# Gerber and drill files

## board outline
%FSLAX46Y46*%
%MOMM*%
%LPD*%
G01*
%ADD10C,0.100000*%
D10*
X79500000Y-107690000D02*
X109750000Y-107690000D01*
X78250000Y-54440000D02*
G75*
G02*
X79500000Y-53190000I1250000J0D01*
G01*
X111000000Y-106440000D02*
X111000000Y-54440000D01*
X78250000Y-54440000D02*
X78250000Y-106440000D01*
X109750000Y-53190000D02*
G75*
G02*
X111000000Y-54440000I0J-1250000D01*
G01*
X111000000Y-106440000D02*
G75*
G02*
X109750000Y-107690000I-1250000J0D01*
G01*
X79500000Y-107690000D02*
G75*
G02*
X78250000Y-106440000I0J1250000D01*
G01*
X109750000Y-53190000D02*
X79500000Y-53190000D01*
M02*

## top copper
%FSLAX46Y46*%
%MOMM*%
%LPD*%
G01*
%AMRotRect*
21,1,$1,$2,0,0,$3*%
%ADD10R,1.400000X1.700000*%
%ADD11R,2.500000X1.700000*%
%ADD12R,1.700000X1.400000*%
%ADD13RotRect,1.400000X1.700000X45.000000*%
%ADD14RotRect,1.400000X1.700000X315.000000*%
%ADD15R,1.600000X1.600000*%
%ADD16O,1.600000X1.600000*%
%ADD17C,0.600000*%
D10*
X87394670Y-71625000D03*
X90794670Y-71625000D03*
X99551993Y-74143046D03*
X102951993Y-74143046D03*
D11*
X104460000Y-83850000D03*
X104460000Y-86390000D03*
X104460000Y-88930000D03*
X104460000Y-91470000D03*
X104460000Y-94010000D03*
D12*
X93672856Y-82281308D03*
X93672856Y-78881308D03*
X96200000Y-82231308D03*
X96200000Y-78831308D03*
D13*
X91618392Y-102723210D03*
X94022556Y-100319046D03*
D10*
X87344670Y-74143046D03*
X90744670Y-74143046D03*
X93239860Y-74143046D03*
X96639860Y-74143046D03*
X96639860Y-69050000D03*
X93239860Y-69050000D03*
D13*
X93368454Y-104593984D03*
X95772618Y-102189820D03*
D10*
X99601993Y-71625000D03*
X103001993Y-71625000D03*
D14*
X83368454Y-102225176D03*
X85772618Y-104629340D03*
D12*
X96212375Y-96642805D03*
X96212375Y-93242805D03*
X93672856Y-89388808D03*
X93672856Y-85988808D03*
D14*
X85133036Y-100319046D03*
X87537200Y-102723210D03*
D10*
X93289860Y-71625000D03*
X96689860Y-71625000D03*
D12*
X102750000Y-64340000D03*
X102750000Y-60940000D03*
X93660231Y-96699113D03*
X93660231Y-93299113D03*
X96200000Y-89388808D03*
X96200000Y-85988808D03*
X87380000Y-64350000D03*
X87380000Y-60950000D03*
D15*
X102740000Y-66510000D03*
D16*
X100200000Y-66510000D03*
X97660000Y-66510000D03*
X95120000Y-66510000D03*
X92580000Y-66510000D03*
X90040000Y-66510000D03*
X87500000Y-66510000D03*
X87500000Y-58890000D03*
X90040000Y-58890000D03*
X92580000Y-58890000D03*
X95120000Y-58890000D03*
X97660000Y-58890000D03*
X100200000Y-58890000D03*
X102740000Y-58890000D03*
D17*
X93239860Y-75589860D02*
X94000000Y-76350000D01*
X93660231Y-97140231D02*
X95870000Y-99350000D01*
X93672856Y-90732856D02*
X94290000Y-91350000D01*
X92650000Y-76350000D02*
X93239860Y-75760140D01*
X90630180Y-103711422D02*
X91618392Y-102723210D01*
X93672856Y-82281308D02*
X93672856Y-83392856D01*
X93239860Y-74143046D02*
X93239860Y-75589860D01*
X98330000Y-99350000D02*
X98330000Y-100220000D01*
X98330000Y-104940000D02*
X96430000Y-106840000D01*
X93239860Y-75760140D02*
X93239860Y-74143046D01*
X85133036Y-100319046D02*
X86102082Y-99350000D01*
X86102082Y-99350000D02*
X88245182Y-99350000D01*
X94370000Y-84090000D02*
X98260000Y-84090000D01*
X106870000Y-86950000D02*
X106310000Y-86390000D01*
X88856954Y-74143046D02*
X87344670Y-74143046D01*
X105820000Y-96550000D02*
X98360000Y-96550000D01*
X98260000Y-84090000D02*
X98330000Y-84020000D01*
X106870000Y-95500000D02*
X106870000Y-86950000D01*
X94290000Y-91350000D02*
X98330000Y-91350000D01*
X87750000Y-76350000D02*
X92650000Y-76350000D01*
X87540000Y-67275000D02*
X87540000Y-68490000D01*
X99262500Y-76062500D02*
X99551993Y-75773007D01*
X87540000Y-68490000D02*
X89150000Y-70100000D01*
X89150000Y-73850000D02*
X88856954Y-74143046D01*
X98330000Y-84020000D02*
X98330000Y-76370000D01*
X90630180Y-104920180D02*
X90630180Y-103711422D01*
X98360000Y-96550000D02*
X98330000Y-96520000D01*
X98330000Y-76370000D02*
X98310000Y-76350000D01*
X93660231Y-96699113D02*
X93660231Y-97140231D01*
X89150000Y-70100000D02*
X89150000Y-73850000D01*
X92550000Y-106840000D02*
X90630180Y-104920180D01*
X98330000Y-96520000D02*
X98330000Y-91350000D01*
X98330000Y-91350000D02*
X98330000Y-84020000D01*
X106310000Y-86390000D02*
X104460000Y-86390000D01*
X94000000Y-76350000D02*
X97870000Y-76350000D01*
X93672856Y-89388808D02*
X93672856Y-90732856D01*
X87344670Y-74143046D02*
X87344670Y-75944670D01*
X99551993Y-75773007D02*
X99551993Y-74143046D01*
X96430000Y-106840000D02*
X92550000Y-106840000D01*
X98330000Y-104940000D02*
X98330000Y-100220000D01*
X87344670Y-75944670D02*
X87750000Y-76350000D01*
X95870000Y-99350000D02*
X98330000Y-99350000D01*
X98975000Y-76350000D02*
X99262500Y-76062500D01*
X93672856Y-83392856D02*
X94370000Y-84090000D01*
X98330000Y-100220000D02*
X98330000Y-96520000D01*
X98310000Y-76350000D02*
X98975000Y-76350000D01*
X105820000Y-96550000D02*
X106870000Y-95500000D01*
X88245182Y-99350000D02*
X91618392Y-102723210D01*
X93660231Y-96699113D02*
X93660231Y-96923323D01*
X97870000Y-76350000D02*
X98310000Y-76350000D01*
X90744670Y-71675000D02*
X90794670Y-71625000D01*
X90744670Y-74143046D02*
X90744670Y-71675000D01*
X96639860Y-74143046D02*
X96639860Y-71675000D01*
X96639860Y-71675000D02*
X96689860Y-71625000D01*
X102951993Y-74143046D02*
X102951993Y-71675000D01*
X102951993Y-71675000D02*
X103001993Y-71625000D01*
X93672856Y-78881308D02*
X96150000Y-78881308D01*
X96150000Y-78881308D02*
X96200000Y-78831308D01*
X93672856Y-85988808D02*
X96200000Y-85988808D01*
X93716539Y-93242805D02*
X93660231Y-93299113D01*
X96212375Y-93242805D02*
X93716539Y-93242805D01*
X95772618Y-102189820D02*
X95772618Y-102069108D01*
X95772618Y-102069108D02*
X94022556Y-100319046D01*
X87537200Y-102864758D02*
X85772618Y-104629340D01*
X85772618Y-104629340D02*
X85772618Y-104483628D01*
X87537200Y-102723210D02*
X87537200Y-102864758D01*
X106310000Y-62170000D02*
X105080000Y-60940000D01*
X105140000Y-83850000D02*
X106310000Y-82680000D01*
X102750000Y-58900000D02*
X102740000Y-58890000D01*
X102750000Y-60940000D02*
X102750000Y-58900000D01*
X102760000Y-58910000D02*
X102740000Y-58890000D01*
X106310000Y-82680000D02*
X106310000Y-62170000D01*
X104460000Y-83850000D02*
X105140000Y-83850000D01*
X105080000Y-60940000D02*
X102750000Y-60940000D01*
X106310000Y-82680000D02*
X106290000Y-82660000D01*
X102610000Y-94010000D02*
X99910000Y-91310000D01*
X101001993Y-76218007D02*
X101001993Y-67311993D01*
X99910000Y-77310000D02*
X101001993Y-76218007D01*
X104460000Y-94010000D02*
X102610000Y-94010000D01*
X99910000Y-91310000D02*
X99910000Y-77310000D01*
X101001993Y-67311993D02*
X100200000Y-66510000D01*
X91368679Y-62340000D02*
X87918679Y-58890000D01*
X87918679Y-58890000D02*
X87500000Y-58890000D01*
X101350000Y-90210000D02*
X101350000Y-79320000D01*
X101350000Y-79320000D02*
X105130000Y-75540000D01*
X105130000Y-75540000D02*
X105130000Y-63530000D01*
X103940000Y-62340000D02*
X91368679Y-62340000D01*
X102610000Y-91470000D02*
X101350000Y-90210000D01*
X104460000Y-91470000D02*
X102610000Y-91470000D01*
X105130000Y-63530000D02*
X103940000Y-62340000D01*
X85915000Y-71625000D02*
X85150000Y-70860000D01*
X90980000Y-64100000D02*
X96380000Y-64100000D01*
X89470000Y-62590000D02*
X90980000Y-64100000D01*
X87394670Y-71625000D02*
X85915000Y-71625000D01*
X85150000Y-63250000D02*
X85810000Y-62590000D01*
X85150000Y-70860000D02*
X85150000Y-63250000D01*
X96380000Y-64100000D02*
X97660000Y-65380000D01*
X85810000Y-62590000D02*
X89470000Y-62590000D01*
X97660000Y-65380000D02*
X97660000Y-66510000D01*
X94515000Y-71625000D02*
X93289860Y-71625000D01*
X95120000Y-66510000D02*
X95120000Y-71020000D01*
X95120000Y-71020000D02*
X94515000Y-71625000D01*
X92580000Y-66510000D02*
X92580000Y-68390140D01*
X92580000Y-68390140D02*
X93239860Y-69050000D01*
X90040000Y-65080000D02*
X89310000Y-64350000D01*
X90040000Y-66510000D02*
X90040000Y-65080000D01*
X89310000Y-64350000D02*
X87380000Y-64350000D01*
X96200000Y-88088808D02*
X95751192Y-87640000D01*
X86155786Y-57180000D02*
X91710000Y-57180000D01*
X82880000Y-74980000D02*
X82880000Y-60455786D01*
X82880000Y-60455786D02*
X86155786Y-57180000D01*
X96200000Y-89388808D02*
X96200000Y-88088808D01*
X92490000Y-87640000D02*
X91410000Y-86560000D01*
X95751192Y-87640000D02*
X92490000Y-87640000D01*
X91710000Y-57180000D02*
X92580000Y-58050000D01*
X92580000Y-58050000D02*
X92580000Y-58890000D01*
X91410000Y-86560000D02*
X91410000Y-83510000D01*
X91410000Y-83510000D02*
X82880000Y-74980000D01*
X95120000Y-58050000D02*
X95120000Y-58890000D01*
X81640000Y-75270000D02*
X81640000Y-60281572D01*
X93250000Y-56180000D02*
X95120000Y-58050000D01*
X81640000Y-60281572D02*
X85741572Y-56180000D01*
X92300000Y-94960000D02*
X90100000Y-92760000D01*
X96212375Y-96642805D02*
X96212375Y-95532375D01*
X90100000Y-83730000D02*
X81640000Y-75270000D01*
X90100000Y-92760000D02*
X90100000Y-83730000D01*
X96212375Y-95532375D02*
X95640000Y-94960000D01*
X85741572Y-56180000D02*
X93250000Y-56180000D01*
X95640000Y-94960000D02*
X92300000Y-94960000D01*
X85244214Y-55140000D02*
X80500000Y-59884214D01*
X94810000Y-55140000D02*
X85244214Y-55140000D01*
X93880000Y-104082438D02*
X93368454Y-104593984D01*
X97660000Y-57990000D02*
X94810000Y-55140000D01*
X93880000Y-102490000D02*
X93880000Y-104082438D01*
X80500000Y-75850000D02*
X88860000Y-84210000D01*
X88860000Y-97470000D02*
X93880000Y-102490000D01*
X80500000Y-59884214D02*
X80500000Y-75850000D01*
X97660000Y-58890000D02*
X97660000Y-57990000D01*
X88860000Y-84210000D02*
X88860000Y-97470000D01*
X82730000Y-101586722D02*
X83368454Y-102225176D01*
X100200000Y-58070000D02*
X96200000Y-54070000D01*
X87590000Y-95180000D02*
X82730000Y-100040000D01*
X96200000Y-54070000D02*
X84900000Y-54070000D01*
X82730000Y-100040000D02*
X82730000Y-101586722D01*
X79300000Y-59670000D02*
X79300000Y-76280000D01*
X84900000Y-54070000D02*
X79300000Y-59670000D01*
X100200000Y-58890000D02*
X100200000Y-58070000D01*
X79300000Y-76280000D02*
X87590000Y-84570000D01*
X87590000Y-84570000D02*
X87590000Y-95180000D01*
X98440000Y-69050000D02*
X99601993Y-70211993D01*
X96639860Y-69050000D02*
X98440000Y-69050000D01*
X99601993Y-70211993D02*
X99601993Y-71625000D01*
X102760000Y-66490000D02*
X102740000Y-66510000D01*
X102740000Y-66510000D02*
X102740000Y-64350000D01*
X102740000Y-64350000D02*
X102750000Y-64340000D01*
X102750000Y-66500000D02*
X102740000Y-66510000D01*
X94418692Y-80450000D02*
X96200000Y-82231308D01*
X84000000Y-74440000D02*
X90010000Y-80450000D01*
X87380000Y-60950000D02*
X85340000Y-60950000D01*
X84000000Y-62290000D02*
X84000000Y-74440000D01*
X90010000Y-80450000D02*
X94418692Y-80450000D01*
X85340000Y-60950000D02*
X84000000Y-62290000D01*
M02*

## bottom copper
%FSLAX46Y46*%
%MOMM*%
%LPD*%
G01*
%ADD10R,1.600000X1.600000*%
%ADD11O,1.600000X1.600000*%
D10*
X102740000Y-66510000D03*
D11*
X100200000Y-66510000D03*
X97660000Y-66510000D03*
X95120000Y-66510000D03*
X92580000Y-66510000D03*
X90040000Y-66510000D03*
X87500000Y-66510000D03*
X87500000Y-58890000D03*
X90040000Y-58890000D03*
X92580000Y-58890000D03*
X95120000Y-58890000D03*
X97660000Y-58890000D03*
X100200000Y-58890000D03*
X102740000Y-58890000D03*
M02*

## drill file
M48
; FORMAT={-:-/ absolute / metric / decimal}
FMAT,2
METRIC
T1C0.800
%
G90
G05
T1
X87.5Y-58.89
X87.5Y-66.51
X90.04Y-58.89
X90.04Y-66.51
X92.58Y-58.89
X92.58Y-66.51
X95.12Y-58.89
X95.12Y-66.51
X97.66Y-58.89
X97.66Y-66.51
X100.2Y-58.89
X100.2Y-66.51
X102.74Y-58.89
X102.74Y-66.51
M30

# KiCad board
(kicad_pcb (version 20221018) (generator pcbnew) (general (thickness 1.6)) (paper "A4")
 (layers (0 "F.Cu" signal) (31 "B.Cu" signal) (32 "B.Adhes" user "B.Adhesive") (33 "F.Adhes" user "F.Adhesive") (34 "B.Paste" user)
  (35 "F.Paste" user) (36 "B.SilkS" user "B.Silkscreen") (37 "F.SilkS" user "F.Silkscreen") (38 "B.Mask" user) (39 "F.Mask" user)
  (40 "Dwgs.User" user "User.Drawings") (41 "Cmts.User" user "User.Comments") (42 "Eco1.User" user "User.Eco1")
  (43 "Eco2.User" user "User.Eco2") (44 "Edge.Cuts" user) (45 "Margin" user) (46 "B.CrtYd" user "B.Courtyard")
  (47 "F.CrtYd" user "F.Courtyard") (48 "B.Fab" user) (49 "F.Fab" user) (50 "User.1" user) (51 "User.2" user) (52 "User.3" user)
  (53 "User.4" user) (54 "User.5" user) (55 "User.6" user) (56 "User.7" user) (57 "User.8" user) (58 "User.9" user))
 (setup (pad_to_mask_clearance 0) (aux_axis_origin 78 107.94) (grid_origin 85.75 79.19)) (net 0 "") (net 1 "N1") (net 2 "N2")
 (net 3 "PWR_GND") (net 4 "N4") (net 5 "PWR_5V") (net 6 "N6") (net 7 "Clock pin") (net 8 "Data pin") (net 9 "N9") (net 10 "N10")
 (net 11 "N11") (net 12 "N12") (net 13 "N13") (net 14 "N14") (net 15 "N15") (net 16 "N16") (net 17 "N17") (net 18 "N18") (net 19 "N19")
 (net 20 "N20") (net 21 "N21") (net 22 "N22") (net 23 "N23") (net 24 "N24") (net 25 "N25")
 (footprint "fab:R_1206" (layer "F.Cu") (at 89.09467 71.625)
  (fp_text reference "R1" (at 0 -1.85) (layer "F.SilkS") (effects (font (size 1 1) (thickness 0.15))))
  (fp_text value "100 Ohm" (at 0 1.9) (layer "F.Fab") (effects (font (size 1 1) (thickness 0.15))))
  (pad "1" smd rect (at -1.7 0) (size 1.4 1.7) (layers "F.Cu" "F.Paste" "F.Mask") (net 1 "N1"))
  (pad "2" smd rect (at 1.7 0) (size 1.4 1.7) (layers "F.Cu" "F.Paste" "F.Mask") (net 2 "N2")))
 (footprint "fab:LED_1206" (layer "F.Cu") (at 101.251993 74.143046)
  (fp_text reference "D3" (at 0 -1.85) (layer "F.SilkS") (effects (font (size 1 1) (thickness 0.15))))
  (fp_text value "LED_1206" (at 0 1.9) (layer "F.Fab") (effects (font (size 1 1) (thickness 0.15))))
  (pad "1" smd rect (at -1.7 0) (size 1.4 1.7) (layers "F.Cu" "F.Paste" "F.Mask") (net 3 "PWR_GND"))
  (pad "2" smd rect (at 1.7 0) (size 1.4 1.7) (layers "F.Cu" "F.Paste" "F.Mask") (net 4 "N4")))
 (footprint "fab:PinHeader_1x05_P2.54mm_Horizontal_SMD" (layer "F.Cu") (at 104.46 83.85)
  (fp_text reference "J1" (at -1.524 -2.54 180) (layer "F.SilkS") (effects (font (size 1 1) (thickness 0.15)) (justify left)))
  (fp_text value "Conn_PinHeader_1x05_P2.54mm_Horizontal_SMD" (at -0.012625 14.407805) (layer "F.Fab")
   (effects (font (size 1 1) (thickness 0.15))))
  (pad "1" smd rect (at 0 0) (size 2.5 1.7) (layers "F.Cu" "F.Paste" "F.Mask") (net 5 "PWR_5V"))
  (pad "2" smd rect (at 0 2.54) (size 2.5 1.7) (layers "F.Cu" "F.Paste" "F.Mask") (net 3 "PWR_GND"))
  (pad "3" smd rect (at 0 5.08) (size 2.5 1.7) (layers "F.Cu" "F.Paste" "F.Mask") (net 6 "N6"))
  (pad "4" smd rect (at 0 7.62) (size 2.5 1.7) (layers "F.Cu" "F.Paste" "F.Mask") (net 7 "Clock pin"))
  (pad "5" smd rect (at 0 10.16) (size 2.5 1.7) (layers "F.Cu" "F.Paste" "F.Mask") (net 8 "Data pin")))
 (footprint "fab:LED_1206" (layer "F.Cu") (at 93.672856 80.581308 90)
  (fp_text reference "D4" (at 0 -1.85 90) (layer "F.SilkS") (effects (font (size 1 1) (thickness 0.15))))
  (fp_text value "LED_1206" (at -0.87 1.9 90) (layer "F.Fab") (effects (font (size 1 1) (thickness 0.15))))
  (pad "1" smd rect (at -1.7 0 90) (size 1.4 1.7) (layers "F.Cu" "F.Paste" "F.Mask") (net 3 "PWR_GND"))
  (pad "2" smd rect (at 1.7 0 90) (size 1.4 1.7) (layers "F.Cu" "F.Paste" "F.Mask") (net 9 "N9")))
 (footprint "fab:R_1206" (layer "F.Cu") (at 96.2 80.531308 90)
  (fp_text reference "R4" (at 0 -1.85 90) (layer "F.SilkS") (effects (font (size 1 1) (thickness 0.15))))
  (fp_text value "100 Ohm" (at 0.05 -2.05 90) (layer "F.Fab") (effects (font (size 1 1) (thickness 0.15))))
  (pad "1" smd rect (at -1.7 0 90) (size 1.4 1.7) (layers "F.Cu" "F.Paste" "F.Mask") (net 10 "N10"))
  (pad "2" smd rect (at 1.7 0 90) (size 1.4 1.7) (layers "F.Cu" "F.Paste" "F.Mask") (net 9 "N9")))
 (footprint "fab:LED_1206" (layer "F.Cu") (at 92.820474 101.521128 45)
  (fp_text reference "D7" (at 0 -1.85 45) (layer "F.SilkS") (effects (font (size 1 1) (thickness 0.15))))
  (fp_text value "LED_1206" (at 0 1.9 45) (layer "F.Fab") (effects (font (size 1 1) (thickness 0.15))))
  (pad "1" smd rect (at -1.7 0 45) (size 1.4 1.7) (layers "F.Cu" "F.Paste" "F.Mask") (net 3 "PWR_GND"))
  (pad "2" smd rect (at 1.7 0 45) (size 1.4 1.7) (layers "F.Cu" "F.Paste" "F.Mask") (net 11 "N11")))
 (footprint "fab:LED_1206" (layer "F.Cu") (at 89.04467 74.143046)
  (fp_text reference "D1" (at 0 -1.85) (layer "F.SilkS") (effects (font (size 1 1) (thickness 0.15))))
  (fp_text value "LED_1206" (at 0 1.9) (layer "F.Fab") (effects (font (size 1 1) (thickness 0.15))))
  (pad "1" smd rect (at -1.7 0) (size 1.4 1.7) (layers "F.Cu" "F.Paste" "F.Mask") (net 3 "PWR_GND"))
  (pad "2" smd rect (at 1.7 0) (size 1.4 1.7) (layers "F.Cu" "F.Paste" "F.Mask") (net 2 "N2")))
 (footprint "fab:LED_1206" (layer "F.Cu") (at 94.93986 74.143046)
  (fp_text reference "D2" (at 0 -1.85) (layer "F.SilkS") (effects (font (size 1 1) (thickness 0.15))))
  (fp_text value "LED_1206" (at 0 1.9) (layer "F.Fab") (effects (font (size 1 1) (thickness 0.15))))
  (pad "1" smd rect (at -1.7 0) (size 1.4 1.7) (layers "F.Cu" "F.Paste" "F.Mask") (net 3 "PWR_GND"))
  (pad "2" smd rect (at 1.7 0) (size 1.4 1.7) (layers "F.Cu" "F.Paste" "F.Mask") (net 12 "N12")))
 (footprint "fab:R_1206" (layer "F.Cu") (at 94.93986 69.05 180)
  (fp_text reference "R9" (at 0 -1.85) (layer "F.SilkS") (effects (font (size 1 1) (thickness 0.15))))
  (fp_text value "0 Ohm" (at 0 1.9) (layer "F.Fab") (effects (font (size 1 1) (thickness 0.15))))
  (pad "1" smd rect (at -1.7 0 180) (size 1.4 1.7) (layers "F.Cu" "F.Paste" "F.Mask") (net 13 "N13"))
  (pad "2" smd rect (at 1.7 0 180) (size 1.4 1.7) (layers "F.Cu" "F.Paste" "F.Mask") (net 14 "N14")))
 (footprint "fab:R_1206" (layer "F.Cu") (at 94.570536 103.391902 45)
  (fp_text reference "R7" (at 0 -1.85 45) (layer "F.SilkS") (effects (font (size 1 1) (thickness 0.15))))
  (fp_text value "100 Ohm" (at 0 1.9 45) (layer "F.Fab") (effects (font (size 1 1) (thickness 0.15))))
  (pad "1" smd rect (at -1.7 0 45) (size 1.4 1.7) (layers "F.Cu" "F.Paste" "F.Mask") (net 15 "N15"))
  (pad "2" smd rect (at 1.7 0 45) (size 1.4 1.7) (layers "F.Cu" "F.Paste" "F.Mask") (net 11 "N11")))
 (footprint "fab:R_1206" (layer "F.Cu") (at 101.301993 71.625)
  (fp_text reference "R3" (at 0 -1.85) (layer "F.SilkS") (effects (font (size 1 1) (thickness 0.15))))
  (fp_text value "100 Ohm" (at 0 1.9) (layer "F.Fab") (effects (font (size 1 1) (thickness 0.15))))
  (pad "1" smd rect (at -1.7 0) (size 1.4 1.7) (layers "F.Cu" "F.Paste" "F.Mask") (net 14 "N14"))
  (pad "2" smd rect (at 1.7 0) (size 1.4 1.7) (layers "F.Cu" "F.Paste" "F.Mask") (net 4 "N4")))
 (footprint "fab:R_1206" (layer "F.Cu") (at 84.570536 103.427258 -45)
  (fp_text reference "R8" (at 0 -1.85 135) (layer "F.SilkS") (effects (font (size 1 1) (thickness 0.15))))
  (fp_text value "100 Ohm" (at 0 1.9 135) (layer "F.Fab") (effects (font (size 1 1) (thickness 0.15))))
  (pad "1" smd rect (at -1.7 0 315) (size 1.4 1.7) (layers "F.Cu" "F.Paste" "F.Mask") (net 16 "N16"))
  (pad "2" smd rect (at 1.7 0 315) (size 1.4 1.7) (layers "F.Cu" "F.Paste" "F.Mask") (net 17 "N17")))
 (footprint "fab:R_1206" (layer "F.Cu") (at 96.212375 94.942805 90)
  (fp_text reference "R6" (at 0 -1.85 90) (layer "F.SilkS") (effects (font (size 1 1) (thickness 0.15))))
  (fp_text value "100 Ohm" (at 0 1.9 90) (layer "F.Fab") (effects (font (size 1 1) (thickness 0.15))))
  (pad "1" smd rect (at -1.7 0 90) (size 1.4 1.7) (layers "F.Cu" "F.Paste" "F.Mask") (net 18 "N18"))
  (pad "2" smd rect (at 1.7 0 90) (size 1.4 1.7) (layers "F.Cu" "F.Paste" "F.Mask") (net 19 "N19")))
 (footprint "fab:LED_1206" (layer "F.Cu") (at 93.672856 87.688808 90)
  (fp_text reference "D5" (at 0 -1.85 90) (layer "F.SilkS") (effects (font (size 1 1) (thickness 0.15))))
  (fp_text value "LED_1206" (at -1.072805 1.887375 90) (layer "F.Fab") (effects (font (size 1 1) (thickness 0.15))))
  (pad "1" smd rect (at -1.7 0 90) (size 1.4 1.7) (layers "F.Cu" "F.Paste" "F.Mask") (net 3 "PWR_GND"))
  (pad "2" smd rect (at 1.7 0 90) (size 1.4 1.7) (layers "F.Cu" "F.Paste" "F.Mask") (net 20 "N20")))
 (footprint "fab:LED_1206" (layer "F.Cu") (at 86.335118 101.521128 -45)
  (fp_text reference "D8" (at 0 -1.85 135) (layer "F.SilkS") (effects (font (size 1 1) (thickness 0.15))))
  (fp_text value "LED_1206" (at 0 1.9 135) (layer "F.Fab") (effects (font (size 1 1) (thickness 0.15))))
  (pad "1" smd rect (at -1.7 0 315) (size 1.4 1.7) (layers "F.Cu" "F.Paste" "F.Mask") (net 3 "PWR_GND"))
  (pad "2" smd rect (at 1.7 0 315) (size 1.4 1.7) (layers "F.Cu" "F.Paste" "F.Mask") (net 17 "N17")))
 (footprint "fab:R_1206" (layer "F.Cu") (at 94.98986 71.625)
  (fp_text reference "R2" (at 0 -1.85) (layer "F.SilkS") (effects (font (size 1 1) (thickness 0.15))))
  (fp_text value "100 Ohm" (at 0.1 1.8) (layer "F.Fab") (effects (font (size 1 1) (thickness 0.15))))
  (pad "1" smd rect (at -1.7 0) (size 1.4 1.7) (layers "F.Cu" "F.Paste" "F.Mask") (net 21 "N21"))
  (pad "2" smd rect (at 1.7 0) (size 1.4 1.7) (layers "F.Cu" "F.Paste" "F.Mask") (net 12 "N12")))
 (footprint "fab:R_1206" (layer "F.Cu") (at 102.75 62.64 90)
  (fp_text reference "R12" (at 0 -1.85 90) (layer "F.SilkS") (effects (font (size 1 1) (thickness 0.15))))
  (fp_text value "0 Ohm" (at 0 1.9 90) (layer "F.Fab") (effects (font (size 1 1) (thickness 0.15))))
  (pad "1" smd rect (at -1.7 0 90) (size 1.4 1.7) (layers "F.Cu" "F.Paste" "F.Mask") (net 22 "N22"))
  (pad "2" smd rect (at 1.7 0 90) (size 1.4 1.7) (layers "F.Cu" "F.Paste" "F.Mask") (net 5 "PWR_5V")))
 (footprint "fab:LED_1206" (layer "F.Cu") (at 93.660231 94.999113 90)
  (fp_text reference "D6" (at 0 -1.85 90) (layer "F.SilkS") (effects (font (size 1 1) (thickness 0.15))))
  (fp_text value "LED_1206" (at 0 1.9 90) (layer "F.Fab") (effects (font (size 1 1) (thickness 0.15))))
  (pad "1" smd rect (at -1.7 0 90) (size 1.4 1.7) (layers "F.Cu" "F.Paste" "F.Mask") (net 3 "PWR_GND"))
  (pad "2" smd rect (at 1.7 0 90) (size 1.4 1.7) (layers "F.Cu" "F.Paste" "F.Mask") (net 19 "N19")))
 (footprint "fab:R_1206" (layer "F.Cu") (at 96.2 87.688808 90)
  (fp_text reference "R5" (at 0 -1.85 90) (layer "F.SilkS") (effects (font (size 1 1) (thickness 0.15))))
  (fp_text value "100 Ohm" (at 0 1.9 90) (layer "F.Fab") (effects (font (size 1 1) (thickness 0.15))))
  (pad "1" smd rect (at -1.7 0 90) (size 1.4 1.7) (layers "F.Cu" "F.Paste" "F.Mask") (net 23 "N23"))
  (pad "2" smd rect (at 1.7 0 90) (size 1.4 1.7) (layers "F.Cu" "F.Paste" "F.Mask") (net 20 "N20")))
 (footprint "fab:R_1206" (layer "F.Cu") (at 87.38 62.65 90)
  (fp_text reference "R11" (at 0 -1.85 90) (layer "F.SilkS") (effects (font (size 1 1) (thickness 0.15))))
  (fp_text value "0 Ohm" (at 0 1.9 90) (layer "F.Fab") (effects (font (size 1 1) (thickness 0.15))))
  (pad "1" smd rect (at -1.7 0 90) (size 1.4 1.7) (layers "F.Cu" "F.Paste" "F.Mask") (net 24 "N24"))
  (pad "2" smd rect (at 1.7 0 90) (size 1.4 1.7) (layers "F.Cu" "F.Paste" "F.Mask") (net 10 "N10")))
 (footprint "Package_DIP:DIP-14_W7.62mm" (layer "B.Cu") (at 102.74 66.51 90)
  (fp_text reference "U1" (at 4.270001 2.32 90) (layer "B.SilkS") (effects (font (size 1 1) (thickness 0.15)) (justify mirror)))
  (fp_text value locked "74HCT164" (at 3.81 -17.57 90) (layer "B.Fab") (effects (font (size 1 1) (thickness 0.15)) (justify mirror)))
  (pad "1" thru_hole rect (at 0 0 90) (size 1.6 1.6) (drill 0.8) (layers "*.Cu" "*.Mask") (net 22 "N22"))
  (pad "2" thru_hole oval (at 0 -2.54 90) (size 1.6 1.6) (drill 0.8) (layers "*.Cu" "*.Mask") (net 8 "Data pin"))
  (pad "3" thru_hole oval (at 0 -5.08 90) (size 1.6 1.6) (drill 0.8) (layers "*.Cu" "*.Mask") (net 1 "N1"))
  (pad "4" thru_hole oval (at 0 -7.62 90) (size 1.6 1.6) (drill 0.8) (layers "*.Cu" "*.Mask") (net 21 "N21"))
  (pad "5" thru_hole oval (at 0 -10.16 90) (size 1.6 1.6) (drill 0.8) (layers "*.Cu" "*.Mask") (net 13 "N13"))
  (pad "6" thru_hole oval (at 0 -12.7 90) (size 1.6 1.6) (drill 0.8) (layers "*.Cu" "*.Mask") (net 24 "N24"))
  (pad "7" thru_hole oval (at 0 -15.24 90) (size 1.6 1.6) (drill 0.8) (layers "*.Cu" "*.Mask") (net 3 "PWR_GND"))
  (pad "8" thru_hole oval (at 7.62 -15.24 90) (size 1.6 1.6) (drill 0.8) (layers "*.Cu" "*.Mask") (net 7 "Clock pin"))
  (pad "9" thru_hole oval (at 7.62 -12.7 90) (size 1.6 1.6) (drill 0.8) (layers "*.Cu" "*.Mask") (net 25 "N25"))
  (pad "10" thru_hole oval (at 7.62 -10.16 90) (size 1.6 1.6) (drill 0.8) (layers "*.Cu" "*.Mask") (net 23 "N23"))
  (pad "11" thru_hole oval (at 7.62 -7.62 90) (size 1.6 1.6) (drill 0.8) (layers "*.Cu" "*.Mask") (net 18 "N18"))
  (pad "12" thru_hole oval (at 7.62 -5.08 90) (size 1.6 1.6) (drill 0.8) (layers "*.Cu" "*.Mask") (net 15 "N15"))
  (pad "13" thru_hole oval (at 7.62 -2.54 90) (size 1.6 1.6) (drill 0.8) (layers "*.Cu" "*.Mask") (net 16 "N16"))
  (pad "14" thru_hole oval (at 7.62 0 90) (size 1.6 1.6) (drill 0.8) (layers "*.Cu" "*.Mask") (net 5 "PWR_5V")))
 (gr_line (start 79.5 107.69) (end 109.75 107.69) (stroke (width 0.1) (type default)) (layer "Edge.Cuts"))
 (gr_arc (start 78.25 54.44) (mid 78.616117 53.556117) (end 79.5 53.19) (stroke (width 0.1) (type default)) (layer "Edge.Cuts"))
 (gr_line (start 111 106.44) (end 111 54.44) (stroke (width 0.1) (type default)) (layer "Edge.Cuts"))
 (gr_line (start 78.25 54.44) (end 78.25 106.44) (stroke (width 0.1) (type default)) (layer "Edge.Cuts"))
 (gr_arc (start 109.75 53.19) (mid 110.633883 53.556117) (end 111 54.44) (stroke (width 0.1) (type default)) (layer "Edge.Cuts"))
 (gr_arc (start 111 106.44) (mid 110.633883 107.323883) (end 109.75 107.69) (stroke (width 0.1) (type default)) (layer "Edge.Cuts"))
 (gr_arc (start 79.5 107.69) (mid 78.616117 107.323883) (end 78.25 106.44) (stroke (width 0.1) (type default)) (layer "Edge.Cuts"))
 (gr_line (start 109.75 53.19) (end 79.5 53.19) (stroke (width 0.1) (type default)) (layer "Edge.Cuts"))
 (segment (start 93.23986 75.58986) (end 94 76.35) (width 0.6) (layer "F.Cu") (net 3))
 (segment (start 93.660231 97.140231) (end 95.87 99.35) (width 0.6) (layer "F.Cu") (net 3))
 (segment (start 93.672856 90.732856) (end 94.29 91.35) (width 0.6) (layer "F.Cu") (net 3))
 (segment (start 92.65 76.35) (end 93.23986 75.76014) (width 0.6) (layer "F.Cu") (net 3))
 (segment (start 90.63018 103.711422) (end 91.618392 102.72321) (width 0.6) (layer "F.Cu") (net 3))
 (segment (start 93.672856 82.281308) (end 93.672856 83.392856) (width 0.6) (layer "F.Cu") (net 3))
 (segment (start 93.23986 74.143046) (end 93.23986 75.58986) (width 0.6) (layer "F.Cu") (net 3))
 (segment (start 98.33 99.35) (end 98.33 100.22) (width 0.6) (layer "F.Cu") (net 3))
 (segment (start 98.33 104.94) (end 96.43 106.84) (width 0.6) (layer "F.Cu") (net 3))
 (segment (start 93.23986 75.76014) (end 93.23986 74.143046) (width 0.6) (layer "F.Cu") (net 3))
 (segment (start 85.133036 100.319046) (end 86.102082 99.35) (width 0.6) (layer "F.Cu") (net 3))
 (segment (start 86.102082 99.35) (end 88.245182 99.35) (width 0.6) (layer "F.Cu") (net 3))
 (segment (start 94.37 84.09) (end 98.26 84.09) (width 0.6) (layer "F.Cu") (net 3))
 (segment (start 106.87 86.95) (end 106.31 86.39) (width 0.6) (layer "F.Cu") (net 3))
 (segment (start 88.856954 74.143046) (end 87.34467 74.143046) (width 0.6) (layer "F.Cu") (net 3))
 (segment (start 105.82 96.55) (end 98.36 96.55) (width 0.6) (layer "F.Cu") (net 3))
 (segment (start 98.26 84.09) (end 98.33 84.02) (width 0.6) (layer "F.Cu") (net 3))
 (segment (start 106.87 95.5) (end 106.87 86.95) (width 0.6) (layer "F.Cu") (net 3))
 (segment (start 94.29 91.35) (end 98.33 91.35) (width 0.6) (layer "F.Cu") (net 3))
 (segment (start 87.75 76.35) (end 92.65 76.35) (width 0.6) (layer "F.Cu") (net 3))
 (segment (start 87.54 67.275) (end 87.54 68.49) (width 0.6) (layer "F.Cu") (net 3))
 (segment (start 99.2625 76.0625) (end 99.551993 75.773007) (width 0.6) (layer "F.Cu") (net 3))
 (segment (start 87.54 68.49) (end 89.15 70.1) (width 0.6) (layer "F.Cu") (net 3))
 (segment (start 89.15 73.85) (end 88.856954 74.143046) (width 0.6) (layer "F.Cu") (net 3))
 (segment (start 98.33 84.02) (end 98.33 76.37) (width 0.6) (layer "F.Cu") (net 3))
 (segment (start 90.63018 104.92018) (end 90.63018 103.711422) (width 0.6) (layer "F.Cu") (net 3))
 (segment (start 98.36 96.55) (end 98.33 96.52) (width 0.6) (layer "F.Cu") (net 3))
 (segment (start 98.33 76.37) (end 98.31 76.35) (width 0.6) (layer "F.Cu") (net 3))
 (segment (start 93.660231 96.699113) (end 93.660231 97.140231) (width 0.6) (layer "F.Cu") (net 3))
 (segment (start 89.15 70.1) (end 89.15 73.85) (width 0.6) (layer "F.Cu") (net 3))
 (segment (start 92.55 106.84) (end 90.63018 104.92018) (width 0.6) (layer "F.Cu") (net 3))
 (segment (start 98.33 96.52) (end 98.33 91.35) (width 0.6) (layer "F.Cu") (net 3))
 (segment (start 98.33 91.35) (end 98.33 84.02) (width 0.6) (layer "F.Cu") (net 3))
 (segment (start 106.31 86.39) (end 104.46 86.39) (width 0.6) (layer "F.Cu") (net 3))
 (segment (start 94 76.35) (end 97.87 76.35) (width 0.6) (layer "F.Cu") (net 3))
 (segment (start 93.672856 89.388808) (end 93.672856 90.732856) (width 0.6) (layer "F.Cu") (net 3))
 (segment (start 87.34467 74.143046) (end 87.34467 75.94467) (width 0.6) (layer "F.Cu") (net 3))
 (segment (start 99.551993 75.773007) (end 99.551993 74.143046) (width 0.6) (layer "F.Cu") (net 3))
 (segment (start 96.43 106.84) (end 92.55 106.84) (width 0.6) (layer "F.Cu") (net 3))
 (segment (start 98.33 104.94) (end 98.33 100.22) (width 0.6) (layer "F.Cu") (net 3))
 (segment (start 87.34467 75.94467) (end 87.75 76.35) (width 0.6) (layer "F.Cu") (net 3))
 (segment (start 95.87 99.35) (end 98.33 99.35) (width 0.6) (layer "F.Cu") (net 3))
 (segment (start 98.975 76.35) (end 99.2625 76.0625) (width 0.6) (layer "F.Cu") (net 3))
 (segment (start 93.672856 83.392856) (end 94.37 84.09) (width 0.6) (layer "F.Cu") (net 3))
 (segment (start 98.33 100.22) (end 98.33 96.52) (width 0.6) (layer "F.Cu") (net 3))
 (segment (start 98.31 76.35) (end 98.975 76.35) (width 0.6) (layer "F.Cu") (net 3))
 (segment (start 105.82 96.55) (end 106.87 95.5) (width 0.6) (layer "F.Cu") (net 3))
 (segment (start 88.245182 99.35) (end 91.618392 102.72321) (width 0.6) (layer "F.Cu") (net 3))
 (segment (start 93.660231 96.699113) (end 93.660231 96.923323) (width 0.6) (layer "F.Cu") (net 3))
 (segment (start 97.87 76.35) (end 98.31 76.35) (width 0.6) (layer "F.Cu") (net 3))
 (segment (start 90.74467 71.675) (end 90.79467 71.625) (width 0.6) (layer "F.Cu") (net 2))
 (segment (start 90.74467 74.143046) (end 90.74467 71.675) (width 0.6) (layer "F.Cu") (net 2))
 (segment (start 96.63986 74.143046) (end 96.63986 71.675) (width 0.6) (layer "F.Cu") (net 12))
 (segment (start 96.63986 71.675) (end 96.68986 71.625) (width 0.6) (layer "F.Cu") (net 12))
 (segment (start 102.951993 74.143046) (end 102.951993 71.675) (width 0.6) (layer "F.Cu") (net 4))
 (segment (start 102.951993 71.675) (end 103.001993 71.625) (width 0.6) (layer "F.Cu") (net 4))
 (segment (start 93.672856 78.881308) (end 96.15 78.881308) (width 0.6) (layer "F.Cu") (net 9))
 (segment (start 96.15 78.881308) (end 96.2 78.831308) (width 0.6) (layer "F.Cu") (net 9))
 (segment (start 93.672856 85.988808) (end 96.2 85.988808) (width 0.6) (layer "F.Cu") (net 20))
 (segment (start 93.716539 93.242805) (end 93.660231 93.299113) (width 0.6) (layer "F.Cu") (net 19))
 (segment (start 96.212375 93.242805) (end 93.716539 93.242805) (width 0.6) (layer "F.Cu") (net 19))
 (segment (start 95.772618 102.18982) (end 95.772618 102.069108) (width 0.6) (layer "F.Cu") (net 11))
 (segment (start 95.772618 102.069108) (end 94.022556 100.319046) (width 0.6) (layer "F.Cu") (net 11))
 (segment (start 87.5372 102.864758) (end 85.772618 104.62934) (width 0.6) (layer "F.Cu") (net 17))
 (segment (start 85.772618 104.62934) (end 85.772618 104.483628) (width 0.6) (layer "F.Cu") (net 17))
 (segment (start 87.5372 102.72321) (end 87.5372 102.864758) (width 0.6) (layer "F.Cu") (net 17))
 (segment (start 106.31 62.17) (end 105.08 60.94) (width 0.6) (layer "F.Cu") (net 5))
 (segment (start 105.14 83.85) (end 106.31 82.68) (width 0.6) (layer "F.Cu") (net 5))
 (segment (start 102.75 58.9) (end 102.74 58.89) (width 0.6) (layer "F.Cu") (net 5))
 (segment (start 102.75 60.94) (end 102.75 58.9) (width 0.6) (layer "F.Cu") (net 5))
 (segment (start 102.76 58.91) (end 102.74 58.89) (width 0.6) (layer "F.Cu") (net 5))
 (segment (start 106.31 82.68) (end 106.31 62.17) (width 0.6) (layer "F.Cu") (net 5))
 (segment (start 104.46 83.85) (end 105.14 83.85) (width 0.6) (layer "F.Cu") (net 5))
 (segment (start 105.08 60.94) (end 102.75 60.94) (width 0.6) (layer "F.Cu") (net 5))
 (segment (start 106.31 82.68) (end 106.29 82.66) (width 0.6) (layer "F.Cu") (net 5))
 (segment (start 102.61 94.01) (end 99.91 91.31) (width 0.6) (layer "F.Cu") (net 8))
 (segment (start 101.001993 76.218007) (end 101.001993 67.311993) (width 0.6) (layer "F.Cu") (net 8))
 (segment (start 99.91 77.31) (end 101.001993 76.218007) (width 0.6) (layer "F.Cu") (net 8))
 (segment (start 104.46 94.01) (end 102.61 94.01) (width 0.6) (layer "F.Cu") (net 8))
 (segment (start 99.91 91.31) (end 99.91 77.31) (width 0.6) (layer "F.Cu") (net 8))
 (segment (start 101.001993 67.311993) (end 100.2 66.51) (width 0.6) (layer "F.Cu") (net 8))
 (segment (start 91.368679 62.34) (end 87.918679 58.89) (width 0.6) (layer "F.Cu") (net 7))
 (segment (start 87.918679 58.89) (end 87.5 58.89) (width 0.6) (layer "F.Cu") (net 7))
 (segment (start 101.35 90.21) (end 101.35 79.32) (width 0.6) (layer "F.Cu") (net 7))
 (segment (start 101.35 79.32) (end 105.13 75.54) (width 0.6) (layer "F.Cu") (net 7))
 (segment (start 105.13 75.54) (end 105.13 63.53) (width 0.6) (layer "F.Cu") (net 7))
 (segment (start 103.94 62.34) (end 91.368679 62.34) (width 0.6) (layer "F.Cu") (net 7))
 (segment (start 102.61 91.47) (end 101.35 90.21) (width 0.6) (layer "F.Cu") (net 7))
 (segment (start 104.46 91.47) (end 102.61 91.47) (width 0.6) (layer "F.Cu") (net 7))
 (segment (start 105.13 63.53) (end 103.94 62.34) (width 0.6) (layer "F.Cu") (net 7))
 (segment (start 85.915 71.625) (end 85.15 70.86) (width 0.6) (layer "F.Cu") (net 1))
 (segment (start 90.98 64.1) (end 96.38 64.1) (width 0.6) (layer "F.Cu") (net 1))
 (segment (start 89.47 62.59) (end 90.98 64.1) (width 0.6) (layer "F.Cu") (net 1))
 (segment (start 87.39467 71.625) (end 85.915 71.625) (width 0.6) (layer "F.Cu") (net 1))
 (segment (start 85.15 63.25) (end 85.81 62.59) (width 0.6) (layer "F.Cu") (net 1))
 (segment (start 85.15 70.86) (end 85.15 63.25) (width 0.6) (layer "F.Cu") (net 1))
 (segment (start 96.38 64.1) (end 97.66 65.38) (width 0.6) (layer "F.Cu") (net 1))
 (segment (start 85.81 62.59) (end 89.47 62.59) (width 0.6) (layer "F.Cu") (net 1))
 (segment (start 97.66 65.38) (end 97.66 66.51) (width 0.6) (layer "F.Cu") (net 1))
 (segment (start 94.515 71.625) (end 93.28986 71.625) (width 0.6) (layer "F.Cu") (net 21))
 (segment (start 95.12 66.51) (end 95.12 71.02) (width 0.6) (layer "F.Cu") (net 21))
 (segment (start 95.12 71.02) (end 94.515 71.625) (width 0.6) (layer "F.Cu") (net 21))
 (segment (start 92.58 66.51) (end 92.58 68.39014) (width 0.6) (layer "F.Cu") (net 13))
 (segment (start 92.58 68.39014) (end 93.23986 69.05) (width 0.6) (layer "F.Cu") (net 13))
 (segment (start 90.04 65.08) (end 89.31 64.35) (width 0.6) (layer "F.Cu") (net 24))
 (segment (start 90.04 66.51) (end 90.04 65.08) (width 0.6) (layer "F.Cu") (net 24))
 (segment (start 89.31 64.35) (end 87.38 64.35) (width 0.6) (layer "F.Cu") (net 24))
 (segment (start 96.2 88.088808) (end 95.751192 87.64) (width 0.6) (layer "F.Cu") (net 23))
 (segment (start 86.155786 57.18) (end 91.71 57.18) (width 0.6) (layer "F.Cu") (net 23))
 (segment (start 82.88 74.98) (end 82.88 60.455786) (width 0.6) (layer "F.Cu") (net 23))
 (segment (start 82.88 60.455786) (end 86.155786 57.18) (width 0.6) (layer "F.Cu") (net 23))
 (segment (start 96.2 89.388808) (end 96.2 88.088808) (width 0.6) (layer "F.Cu") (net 23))
 (segment (start 92.49 87.64) (end 91.41 86.56) (width 0.6) (layer "F.Cu") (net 23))
 (segment (start 95.751192 87.64) (end 92.49 87.64) (width 0.6) (layer "F.Cu") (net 23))
 (segment (start 91.71 57.18) (end 92.58 58.05) (width 0.6) (layer "F.Cu") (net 23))
 (segment (start 92.58 58.05) (end 92.58 58.89) (width 0.6) (layer "F.Cu") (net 23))
 (segment (start 91.41 86.56) (end 91.41 83.51) (width 0.6) (layer "F.Cu") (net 23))
 (segment (start 91.41 83.51) (end 82.88 74.98) (width 0.6) (layer "F.Cu") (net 23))
 (segment (start 95.12 58.05) (end 95.12 58.89) (width 0.6) (layer "F.Cu") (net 18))
 (segment (start 81.64 75.27) (end 81.64 60.281572) (width 0.6) (layer "F.Cu") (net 18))
 (segment (start 93.25 56.18) (end 95.12 58.05) (width 0.6) (layer "F.Cu") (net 18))
 (segment (start 81.64 60.281572) (end 85.741572 56.18) (width 0.6) (layer "F.Cu") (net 18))
 (segment (start 92.3 94.96) (end 90.1 92.76) (width 0.6) (layer "F.Cu") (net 18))
 (segment (start 96.212375 96.642805) (end 96.212375 95.532375) (width 0.6) (layer "F.Cu") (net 18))
 (segment (start 90.1 83.73) (end 81.64 75.27) (width 0.6) (layer "F.Cu") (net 18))
 (segment (start 90.1 92.76) (end 90.1 83.73) (width 0.6) (layer "F.Cu") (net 18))
 (segment (start 96.212375 95.532375) (end 95.64 94.96) (width 0.6) (layer "F.Cu") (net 18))
 (segment (start 85.741572 56.18) (end 93.25 56.18) (width 0.6) (layer "F.Cu") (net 18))
 (segment (start 95.64 94.96) (end 92.3 94.96) (width 0.6) (layer "F.Cu") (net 18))
 (segment (start 85.244214 55.14) (end 80.5 59.884214) (width 0.6) (layer "F.Cu") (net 15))
 (segment (start 94.81 55.14) (end 85.244214 55.14) (width 0.6) (layer "F.Cu") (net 15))
 (segment (start 93.88 104.082438) (end 93.368454 104.593984) (width 0.6) (layer "F.Cu") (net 15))
 (segment (start 97.66 57.99) (end 94.81 55.14) (width 0.6) (layer "F.Cu") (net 15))
 (segment (start 93.88 102.49) (end 93.88 104.082438) (width 0.6) (layer "F.Cu") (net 15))
 (segment (start 80.5 75.85) (end 88.86 84.21) (width 0.6) (layer "F.Cu") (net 15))
 (segment (start 88.86 97.47) (end 93.88 102.49) (width 0.6) (layer "F.Cu") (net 15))
 (segment (start 80.5 59.884214) (end 80.5 75.85) (width 0.6) (layer "F.Cu") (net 15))
 (segment (start 97.66 58.89) (end 97.66 57.99) (width 0.6) (layer "F.Cu") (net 15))
 (segment (start 88.86 84.21) (end 88.86 97.47) (width 0.6) (layer "F.Cu") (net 15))
 (segment (start 82.73 101.586722) (end 83.368454 102.225176) (width 0.6) (layer "F.Cu") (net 16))
 (segment (start 100.2 58.07) (end 96.2 54.07) (width 0.6) (layer "F.Cu") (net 16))
 (segment (start 87.59 95.18) (end 82.73 100.04) (width 0.6) (layer "F.Cu") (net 16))
 (segment (start 96.2 54.07) (end 84.9 54.07) (width 0.6) (layer "F.Cu") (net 16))
 (segment (start 82.73 100.04) (end 82.73 101.586722) (width 0.6) (layer "F.Cu") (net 16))
 (segment (start 79.3 59.67) (end 79.3 76.28) (width 0.6) (layer "F.Cu") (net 16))
 (segment (start 84.9 54.07) (end 79.3 59.67) (width 0.6) (layer "F.Cu") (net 16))
 (segment (start 100.2 58.89) (end 100.2 58.07) (width 0.6) (layer "F.Cu") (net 16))
 (segment (start 79.3 76.28) (end 87.59 84.57) (width 0.6) (layer "F.Cu") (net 16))
 (segment (start 87.59 84.57) (end 87.59 95.18) (width 0.6) (layer "F.Cu") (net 16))
 (segment (start 98.44 69.05) (end 99.601993 70.211993) (width 0.6) (layer "F.Cu") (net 14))
 (segment (start 96.63986 69.05) (end 98.44 69.05) (width 0.6) (layer "F.Cu") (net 14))
 (segment (start 99.601993 70.211993) (end 99.601993 71.625) (width 0.6) (layer "F.Cu") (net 14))
 (segment (start 102.76 66.49) (end 102.74 66.51) (width 0.6) (layer "F.Cu") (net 22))
 (segment (start 102.74 66.51) (end 102.74 64.35) (width 0.6) (layer "F.Cu") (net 22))
 (segment (start 102.74 64.35) (end 102.75 64.34) (width 0.6) (layer "F.Cu") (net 22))
 (segment (start 102.75 66.5) (end 102.74 66.51) (width 0.6) (layer "F.Cu") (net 22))
 (segment (start 94.418692 80.45) (end 96.2 82.231308) (width 0.6) (layer "F.Cu") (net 10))
 (segment (start 84 74.44) (end 90.01 80.45) (width 0.6) (layer "F.Cu") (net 10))
 (segment (start 87.38 60.95) (end 85.34 60.95) (width 0.6) (layer "F.Cu") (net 10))
 (segment (start 84 62.29) (end 84 74.44) (width 0.6) (layer "F.Cu") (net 10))
 (segment (start 90.01 80.45) (end 94.418692 80.45) (width 0.6) (layer "F.Cu") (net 10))
 (segment (start 85.34 60.95) (end 84 62.29) (width 0.6) (layer "F.Cu") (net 10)))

